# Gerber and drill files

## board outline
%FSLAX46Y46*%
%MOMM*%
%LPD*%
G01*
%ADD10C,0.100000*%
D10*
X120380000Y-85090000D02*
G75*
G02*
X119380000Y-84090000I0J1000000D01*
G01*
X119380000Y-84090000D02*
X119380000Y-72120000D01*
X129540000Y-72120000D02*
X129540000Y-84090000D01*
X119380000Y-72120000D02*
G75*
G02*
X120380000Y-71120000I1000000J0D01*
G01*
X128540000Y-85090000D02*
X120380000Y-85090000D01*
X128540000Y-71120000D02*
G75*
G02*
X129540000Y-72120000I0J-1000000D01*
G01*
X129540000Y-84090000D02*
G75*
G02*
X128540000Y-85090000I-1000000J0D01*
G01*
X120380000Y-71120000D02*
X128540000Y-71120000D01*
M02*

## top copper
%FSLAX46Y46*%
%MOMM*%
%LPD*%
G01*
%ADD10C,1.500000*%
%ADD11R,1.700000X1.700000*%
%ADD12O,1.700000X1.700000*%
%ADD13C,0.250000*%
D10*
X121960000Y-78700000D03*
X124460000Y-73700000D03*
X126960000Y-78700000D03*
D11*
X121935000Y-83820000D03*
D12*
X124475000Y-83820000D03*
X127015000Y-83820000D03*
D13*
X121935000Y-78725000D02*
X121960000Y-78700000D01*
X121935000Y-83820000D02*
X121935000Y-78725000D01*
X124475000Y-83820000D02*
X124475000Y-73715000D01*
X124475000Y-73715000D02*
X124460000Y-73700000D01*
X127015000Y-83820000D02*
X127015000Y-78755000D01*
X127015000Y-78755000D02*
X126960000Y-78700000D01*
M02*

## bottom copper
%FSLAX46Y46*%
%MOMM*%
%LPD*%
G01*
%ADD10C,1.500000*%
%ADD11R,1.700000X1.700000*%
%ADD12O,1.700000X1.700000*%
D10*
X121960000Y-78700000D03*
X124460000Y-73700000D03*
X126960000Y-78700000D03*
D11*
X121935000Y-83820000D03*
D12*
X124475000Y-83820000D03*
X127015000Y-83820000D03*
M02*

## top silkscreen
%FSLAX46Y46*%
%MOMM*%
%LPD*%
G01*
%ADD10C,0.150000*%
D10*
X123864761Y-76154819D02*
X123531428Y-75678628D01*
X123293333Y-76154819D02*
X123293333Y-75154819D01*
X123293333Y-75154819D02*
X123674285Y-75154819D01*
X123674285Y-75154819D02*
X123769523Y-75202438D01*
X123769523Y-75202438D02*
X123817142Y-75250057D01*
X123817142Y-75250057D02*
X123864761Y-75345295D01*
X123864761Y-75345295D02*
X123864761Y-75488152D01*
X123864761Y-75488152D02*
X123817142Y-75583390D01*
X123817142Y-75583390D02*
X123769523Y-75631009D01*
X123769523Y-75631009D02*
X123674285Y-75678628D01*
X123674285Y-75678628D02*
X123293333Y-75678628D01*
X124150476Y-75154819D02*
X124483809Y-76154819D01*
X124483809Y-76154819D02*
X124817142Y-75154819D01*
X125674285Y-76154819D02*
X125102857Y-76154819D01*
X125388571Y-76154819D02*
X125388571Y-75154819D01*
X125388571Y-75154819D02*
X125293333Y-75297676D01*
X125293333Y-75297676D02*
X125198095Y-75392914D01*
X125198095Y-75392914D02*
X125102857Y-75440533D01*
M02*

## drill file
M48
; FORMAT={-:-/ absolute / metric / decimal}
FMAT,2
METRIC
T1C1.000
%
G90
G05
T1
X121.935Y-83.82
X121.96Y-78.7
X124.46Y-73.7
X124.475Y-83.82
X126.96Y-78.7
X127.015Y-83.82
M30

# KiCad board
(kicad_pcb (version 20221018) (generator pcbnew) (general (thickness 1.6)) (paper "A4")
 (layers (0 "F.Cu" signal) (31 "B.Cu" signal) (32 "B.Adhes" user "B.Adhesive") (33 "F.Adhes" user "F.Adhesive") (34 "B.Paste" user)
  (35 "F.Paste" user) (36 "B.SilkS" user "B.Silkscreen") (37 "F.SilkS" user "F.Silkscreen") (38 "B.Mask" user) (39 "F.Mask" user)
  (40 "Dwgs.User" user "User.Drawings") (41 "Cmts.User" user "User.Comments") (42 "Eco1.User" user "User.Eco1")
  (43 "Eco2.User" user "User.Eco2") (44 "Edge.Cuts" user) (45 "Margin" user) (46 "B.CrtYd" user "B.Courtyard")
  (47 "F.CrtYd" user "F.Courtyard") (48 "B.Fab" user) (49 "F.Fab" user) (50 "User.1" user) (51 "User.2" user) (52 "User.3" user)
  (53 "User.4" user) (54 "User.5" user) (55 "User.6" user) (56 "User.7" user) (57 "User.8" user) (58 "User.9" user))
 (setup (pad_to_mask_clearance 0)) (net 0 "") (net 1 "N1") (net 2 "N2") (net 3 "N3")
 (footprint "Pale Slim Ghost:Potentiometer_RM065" (layer "F.Cu") (at 124.46 76.2)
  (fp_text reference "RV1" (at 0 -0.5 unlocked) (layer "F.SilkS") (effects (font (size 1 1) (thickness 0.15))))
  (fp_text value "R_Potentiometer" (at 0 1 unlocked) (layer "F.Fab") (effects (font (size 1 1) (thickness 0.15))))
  (pad "1" thru_hole circle (at -2.5 2.5) (size 1.5 1.5) (drill 1) (layers "*.Cu" "*.Mask") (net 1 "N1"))
  (pad "2" thru_hole circle (at 0 -2.5) (size 1.5 1.5) (drill 1) (layers "*.Cu" "*.Mask") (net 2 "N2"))
  (pad "3" thru_hole circle (at 2.5 2.5) (size 1.5 1.5) (drill 1) (layers "*.Cu" "*.Mask") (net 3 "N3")))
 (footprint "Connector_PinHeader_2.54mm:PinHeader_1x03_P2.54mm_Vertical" (layer "B.Cu") (at 121.935 83.82 -90)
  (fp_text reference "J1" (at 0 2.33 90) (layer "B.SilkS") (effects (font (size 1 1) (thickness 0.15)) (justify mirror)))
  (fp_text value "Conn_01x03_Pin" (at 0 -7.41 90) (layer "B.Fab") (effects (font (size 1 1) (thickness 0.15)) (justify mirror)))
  (pad "1" thru_hole rect (at 0 0 270) (size 1.7 1.7) (drill 1) (layers "*.Cu" "*.Mask") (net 1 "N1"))
  (pad "2" thru_hole oval (at 0 -2.54 270) (size 1.7 1.7) (drill 1) (layers "*.Cu" "*.Mask") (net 2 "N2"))
  (pad "3" thru_hole oval (at 0 -5.08 270) (size 1.7 1.7) (drill 1) (layers "*.Cu" "*.Mask") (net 3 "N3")))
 (gr_arc (start 120.38 85.09) (mid 119.672893 84.797107) (end 119.38 84.09) (stroke (width 0.1) (type default)) (layer "Edge.Cuts"))
 (gr_line (start 119.38 84.09) (end 119.38 72.12) (stroke (width 0.1) (type default)) (layer "Edge.Cuts"))
 (gr_line (start 129.54 72.12) (end 129.54 84.09) (stroke (width 0.1) (type default)) (layer "Edge.Cuts"))
 (gr_arc (start 119.38 72.12) (mid 119.672893 71.412893) (end 120.38 71.12) (stroke (width 0.1) (type default)) (layer "Edge.Cuts"))
 (gr_line (start 128.54 85.09) (end 120.38 85.09) (stroke (width 0.1) (type default)) (layer "Edge.Cuts"))
 (gr_arc (start 128.54 71.12) (mid 129.247107 71.412893) (end 129.54 72.12) (stroke (width 0.1) (type default)) (layer "Edge.Cuts"))
 (gr_arc (start 129.54 84.09) (mid 129.247107 84.797107) (end 128.54 85.09) (stroke (width 0.1) (type default)) (layer "Edge.Cuts"))
 (gr_line (start 120.38 71.12) (end 128.54 71.12) (stroke (width 0.1) (type default)) (layer "Edge.Cuts"))
 (segment (start 121.935 78.725) (end 121.96 78.7) (width 0.25) (layer "F.Cu") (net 1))
 (segment (start 121.935 83.82) (end 121.935 78.725) (width 0.25) (layer "F.Cu") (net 1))
 (segment (start 124.475 83.82) (end 124.475 73.715) (width 0.25) (layer "F.Cu") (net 2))
 (segment (start 124.475 73.715) (end 124.46 73.7) (width 0.25) (layer "F.Cu") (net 2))
 (segment (start 127.015 83.82) (end 127.015 78.755) (width 0.25) (layer "F.Cu") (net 3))
 (segment (start 127.015 78.755) (end 126.96 78.7) (width 0.25) (layer "F.Cu") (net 3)))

